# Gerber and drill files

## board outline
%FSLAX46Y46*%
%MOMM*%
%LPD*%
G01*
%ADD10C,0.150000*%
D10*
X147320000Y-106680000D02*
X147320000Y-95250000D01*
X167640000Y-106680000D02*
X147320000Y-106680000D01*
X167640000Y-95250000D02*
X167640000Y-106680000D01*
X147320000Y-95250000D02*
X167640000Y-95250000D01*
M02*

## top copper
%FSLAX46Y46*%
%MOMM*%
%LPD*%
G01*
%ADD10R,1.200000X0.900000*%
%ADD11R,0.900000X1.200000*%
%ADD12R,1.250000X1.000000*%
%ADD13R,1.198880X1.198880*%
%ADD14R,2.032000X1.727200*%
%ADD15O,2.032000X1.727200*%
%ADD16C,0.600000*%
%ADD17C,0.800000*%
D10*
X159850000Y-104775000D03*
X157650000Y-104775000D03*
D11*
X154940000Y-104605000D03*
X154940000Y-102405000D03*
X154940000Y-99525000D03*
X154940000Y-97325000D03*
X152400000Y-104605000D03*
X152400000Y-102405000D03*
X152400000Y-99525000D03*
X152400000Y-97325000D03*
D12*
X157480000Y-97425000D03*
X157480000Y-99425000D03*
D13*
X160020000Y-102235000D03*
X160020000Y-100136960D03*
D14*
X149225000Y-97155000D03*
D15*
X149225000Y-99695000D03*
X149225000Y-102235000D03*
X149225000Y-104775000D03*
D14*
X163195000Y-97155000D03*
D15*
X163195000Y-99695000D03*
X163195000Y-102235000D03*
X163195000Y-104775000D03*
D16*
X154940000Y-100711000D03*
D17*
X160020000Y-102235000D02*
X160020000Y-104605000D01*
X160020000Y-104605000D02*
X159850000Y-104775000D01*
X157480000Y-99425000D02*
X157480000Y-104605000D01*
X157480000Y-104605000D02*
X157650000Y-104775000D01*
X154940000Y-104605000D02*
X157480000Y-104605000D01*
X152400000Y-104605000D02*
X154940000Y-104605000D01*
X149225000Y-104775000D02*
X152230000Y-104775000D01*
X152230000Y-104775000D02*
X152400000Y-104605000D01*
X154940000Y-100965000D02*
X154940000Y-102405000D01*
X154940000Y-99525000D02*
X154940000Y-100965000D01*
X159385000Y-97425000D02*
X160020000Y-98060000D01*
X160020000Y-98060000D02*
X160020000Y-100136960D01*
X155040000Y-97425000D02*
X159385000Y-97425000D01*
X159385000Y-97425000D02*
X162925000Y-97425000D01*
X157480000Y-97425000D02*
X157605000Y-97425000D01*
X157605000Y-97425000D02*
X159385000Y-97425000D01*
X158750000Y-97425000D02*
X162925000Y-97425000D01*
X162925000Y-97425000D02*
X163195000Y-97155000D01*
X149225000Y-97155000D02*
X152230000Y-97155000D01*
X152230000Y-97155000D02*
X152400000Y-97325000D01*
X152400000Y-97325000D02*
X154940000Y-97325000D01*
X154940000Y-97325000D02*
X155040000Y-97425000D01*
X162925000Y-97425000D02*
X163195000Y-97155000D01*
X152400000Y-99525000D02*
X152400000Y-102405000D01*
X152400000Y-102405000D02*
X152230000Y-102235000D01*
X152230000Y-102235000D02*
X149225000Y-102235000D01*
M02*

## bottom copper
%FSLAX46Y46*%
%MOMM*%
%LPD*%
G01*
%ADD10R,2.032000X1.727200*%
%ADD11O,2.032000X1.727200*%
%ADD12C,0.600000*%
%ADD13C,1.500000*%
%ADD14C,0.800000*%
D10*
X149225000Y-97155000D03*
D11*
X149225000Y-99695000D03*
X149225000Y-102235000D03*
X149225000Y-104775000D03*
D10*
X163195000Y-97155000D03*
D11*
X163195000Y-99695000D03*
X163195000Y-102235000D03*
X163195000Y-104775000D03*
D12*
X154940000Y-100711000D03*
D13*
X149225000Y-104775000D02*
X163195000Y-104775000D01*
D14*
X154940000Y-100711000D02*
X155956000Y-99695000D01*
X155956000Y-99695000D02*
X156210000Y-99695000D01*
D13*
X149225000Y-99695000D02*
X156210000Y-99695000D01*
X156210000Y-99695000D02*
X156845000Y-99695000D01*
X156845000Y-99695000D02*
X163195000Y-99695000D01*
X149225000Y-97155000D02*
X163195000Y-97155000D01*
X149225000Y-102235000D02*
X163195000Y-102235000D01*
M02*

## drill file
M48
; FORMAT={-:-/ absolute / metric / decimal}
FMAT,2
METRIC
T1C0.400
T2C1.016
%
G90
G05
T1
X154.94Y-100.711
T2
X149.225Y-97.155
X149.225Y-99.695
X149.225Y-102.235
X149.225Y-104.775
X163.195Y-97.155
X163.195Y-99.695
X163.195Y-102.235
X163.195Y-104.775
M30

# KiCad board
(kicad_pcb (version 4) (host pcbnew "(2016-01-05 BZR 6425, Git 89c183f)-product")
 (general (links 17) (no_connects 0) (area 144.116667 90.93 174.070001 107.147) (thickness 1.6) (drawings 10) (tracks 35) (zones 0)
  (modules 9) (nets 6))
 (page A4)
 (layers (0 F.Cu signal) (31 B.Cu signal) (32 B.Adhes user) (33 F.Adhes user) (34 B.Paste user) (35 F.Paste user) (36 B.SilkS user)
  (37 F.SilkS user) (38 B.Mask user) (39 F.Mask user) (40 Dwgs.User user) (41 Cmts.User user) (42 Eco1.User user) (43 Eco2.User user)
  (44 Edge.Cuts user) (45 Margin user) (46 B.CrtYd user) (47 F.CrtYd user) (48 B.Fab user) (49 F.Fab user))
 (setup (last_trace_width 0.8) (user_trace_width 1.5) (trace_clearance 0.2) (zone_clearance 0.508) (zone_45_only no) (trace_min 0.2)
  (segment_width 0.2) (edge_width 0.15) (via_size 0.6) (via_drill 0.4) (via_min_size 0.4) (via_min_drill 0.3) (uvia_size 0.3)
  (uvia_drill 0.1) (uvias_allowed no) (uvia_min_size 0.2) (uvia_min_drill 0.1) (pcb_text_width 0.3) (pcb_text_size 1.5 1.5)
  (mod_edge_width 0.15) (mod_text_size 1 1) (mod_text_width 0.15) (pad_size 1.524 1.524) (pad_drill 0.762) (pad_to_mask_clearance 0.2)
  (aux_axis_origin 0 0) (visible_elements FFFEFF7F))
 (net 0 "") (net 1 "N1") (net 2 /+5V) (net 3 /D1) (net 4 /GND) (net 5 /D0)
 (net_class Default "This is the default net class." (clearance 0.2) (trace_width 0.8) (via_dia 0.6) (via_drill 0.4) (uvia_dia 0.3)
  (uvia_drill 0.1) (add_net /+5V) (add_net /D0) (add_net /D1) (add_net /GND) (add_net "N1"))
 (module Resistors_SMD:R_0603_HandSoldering (layer F.Cu) (at 158.75 104.775 180)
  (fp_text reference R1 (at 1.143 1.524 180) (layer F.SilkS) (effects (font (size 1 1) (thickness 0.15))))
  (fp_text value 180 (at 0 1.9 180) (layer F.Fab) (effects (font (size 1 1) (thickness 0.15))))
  (pad 1 smd rect (at -1.1 0 180) (size 1.2 0.9) (layers F.Cu F.Paste F.Mask) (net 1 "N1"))
  (pad 2 smd rect (at 1.1 0 180) (size 1.2 0.9) (layers F.Cu F.Paste F.Mask) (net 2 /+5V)))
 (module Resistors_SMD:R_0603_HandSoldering (layer F.Cu) (at 154.94 103.505 90)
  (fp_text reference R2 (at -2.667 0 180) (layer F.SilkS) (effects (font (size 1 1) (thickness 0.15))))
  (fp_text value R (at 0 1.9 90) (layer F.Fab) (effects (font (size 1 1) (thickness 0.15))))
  (pad 1 smd rect (at -1.1 0 90) (size 1.2 0.9) (layers F.Cu F.Paste F.Mask) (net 2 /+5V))
  (pad 2 smd rect (at 1.1 0 90) (size 1.2 0.9) (layers F.Cu F.Paste F.Mask) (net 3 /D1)))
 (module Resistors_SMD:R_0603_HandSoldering (layer F.Cu) (at 154.94 98.425 90)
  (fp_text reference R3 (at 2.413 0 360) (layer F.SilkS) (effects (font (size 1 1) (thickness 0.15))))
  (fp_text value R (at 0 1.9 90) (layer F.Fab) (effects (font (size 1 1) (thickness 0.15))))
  (pad 1 smd rect (at -1.1 0 90) (size 1.2 0.9) (layers F.Cu F.Paste F.Mask) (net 3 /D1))
  (pad 2 smd rect (at 1.1 0 90) (size 1.2 0.9) (layers F.Cu F.Paste F.Mask) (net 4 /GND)))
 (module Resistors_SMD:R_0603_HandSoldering (layer F.Cu) (at 152.4 103.505 90)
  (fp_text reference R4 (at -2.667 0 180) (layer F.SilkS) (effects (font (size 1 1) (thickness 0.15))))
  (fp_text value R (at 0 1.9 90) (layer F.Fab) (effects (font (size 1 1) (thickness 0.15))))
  (pad 1 smd rect (at -1.1 0 90) (size 1.2 0.9) (layers F.Cu F.Paste F.Mask) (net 2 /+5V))
  (pad 2 smd rect (at 1.1 0 90) (size 1.2 0.9) (layers F.Cu F.Paste F.Mask) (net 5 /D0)))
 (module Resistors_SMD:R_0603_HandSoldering (layer F.Cu) (at 152.4 98.425 90)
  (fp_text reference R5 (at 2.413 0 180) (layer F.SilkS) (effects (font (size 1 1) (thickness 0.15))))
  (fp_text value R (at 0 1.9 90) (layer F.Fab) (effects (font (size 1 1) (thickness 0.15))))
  (pad 1 smd rect (at -1.1 0 90) (size 1.2 0.9) (layers F.Cu F.Paste F.Mask) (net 5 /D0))
  (pad 2 smd rect (at 1.1 0 90) (size 1.2 0.9) (layers F.Cu F.Paste F.Mask) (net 4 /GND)))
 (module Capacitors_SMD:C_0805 (layer F.Cu) (at 157.48 98.425 270)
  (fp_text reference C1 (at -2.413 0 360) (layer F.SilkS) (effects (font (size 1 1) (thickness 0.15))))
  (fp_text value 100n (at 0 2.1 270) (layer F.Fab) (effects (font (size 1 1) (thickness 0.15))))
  (pad 1 smd rect (at -1 0 270) (size 1 1.25) (layers F.Cu F.Paste F.Mask) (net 4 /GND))
  (pad 2 smd rect (at 1 0 270) (size 1 1.25) (layers F.Cu F.Paste F.Mask) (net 2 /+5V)))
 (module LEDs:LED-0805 (layer F.Cu) (at 160.02 101.18598 270)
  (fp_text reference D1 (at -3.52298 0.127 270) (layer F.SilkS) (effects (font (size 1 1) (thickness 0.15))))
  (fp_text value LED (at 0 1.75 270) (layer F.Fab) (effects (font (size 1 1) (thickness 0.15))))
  (pad 2 smd rect (at 1.04902 0 90) (size 1.19888 1.19888) (layers F.Cu F.Paste F.Mask) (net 1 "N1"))
  (pad 1 smd rect (at -1.04902 0 90) (size 1.19888 1.19888) (layers F.Cu F.Paste F.Mask) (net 4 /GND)))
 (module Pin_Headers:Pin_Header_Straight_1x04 (layer F.Cu) (at 149.225 97.155)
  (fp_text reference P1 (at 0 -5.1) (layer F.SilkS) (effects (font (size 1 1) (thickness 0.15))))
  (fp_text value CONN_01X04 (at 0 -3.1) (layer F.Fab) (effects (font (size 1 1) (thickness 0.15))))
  (pad 1 thru_hole rect (at 0 0) (size 2.032 1.7272) (drill 1.016) (layers *.Cu *.Mask F.SilkS) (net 4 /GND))
  (pad 2 thru_hole oval (at 0 2.54) (size 2.032 1.7272) (drill 1.016) (layers *.Cu *.Mask F.SilkS) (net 3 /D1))
  (pad 3 thru_hole oval (at 0 5.08) (size 2.032 1.7272) (drill 1.016) (layers *.Cu *.Mask F.SilkS) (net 5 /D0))
  (pad 4 thru_hole oval (at 0 7.62) (size 2.032 1.7272) (drill 1.016) (layers *.Cu *.Mask F.SilkS) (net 2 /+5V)))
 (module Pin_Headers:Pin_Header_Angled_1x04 (layer F.Cu) (at 163.195 97.155)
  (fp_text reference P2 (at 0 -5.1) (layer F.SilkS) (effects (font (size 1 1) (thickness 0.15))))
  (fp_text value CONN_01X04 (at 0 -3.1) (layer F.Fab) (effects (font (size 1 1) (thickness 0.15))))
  (pad 1 thru_hole rect (at 0 0) (size 2.032 1.7272) (drill 1.016) (layers *.Cu *.Mask F.SilkS) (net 4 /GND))
  (pad 2 thru_hole oval (at 0 2.54) (size 2.032 1.7272) (drill 1.016) (layers *.Cu *.Mask F.SilkS) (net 3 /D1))
  (pad 3 thru_hole oval (at 0 5.08) (size 2.032 1.7272) (drill 1.016) (layers *.Cu *.Mask F.SilkS) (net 5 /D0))
  (pad 4 thru_hole oval (at 0 7.62) (size 2.032 1.7272) (drill 1.016) (layers *.Cu *.Mask F.SilkS) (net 2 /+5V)))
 (gr_line (start 147.32 106.68) (end 147.32 95.25) (layer Edge.Cuts) (width 0.15))
 (gr_line (start 167.64 106.68) (end 147.32 106.68) (layer Edge.Cuts) (width 0.15))
 (gr_line (start 167.64 95.25) (end 167.64 106.68) (layer Edge.Cuts) (width 0.15))
 (gr_line (start 147.32 95.25) (end 167.64 95.25) (layer Edge.Cuts) (width 0.15))
 (segment (start 160.02 102.235) (end 160.02 104.605) (width 0.8) (layer F.Cu) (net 1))
 (segment (start 160.02 104.605) (end 159.85 104.775) (width 0.8) (layer F.Cu) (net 1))
 (segment (start 157.48 99.425) (end 157.48 104.605) (width 0.8) (layer F.Cu) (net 2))
 (segment (start 157.48 104.605) (end 157.65 104.775) (width 0.8) (layer F.Cu) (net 2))
 (segment (start 154.94 104.605) (end 157.48 104.605) (width 0.8) (layer F.Cu) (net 2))
 (segment (start 152.4 104.605) (end 154.94 104.605) (width 0.8) (layer F.Cu) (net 2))
 (segment (start 149.225 104.775) (end 152.23 104.775) (width 0.8) (layer F.Cu) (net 2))
 (segment (start 152.23 104.775) (end 152.4 104.605) (width 0.8) (layer F.Cu) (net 2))
 (segment (start 149.225 104.775) (end 163.195 104.775) (width 1.5) (layer B.Cu) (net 2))
 (segment (start 154.94 100.711) (end 155.956 99.695) (width 0.8) (layer B.Cu) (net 3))
 (segment (start 155.956 99.695) (end 156.21 99.695) (width 0.8) (layer B.Cu) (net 3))
 (segment (start 149.225 99.695) (end 156.21 99.695) (width 1.5) (layer B.Cu) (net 3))
 (segment (start 156.21 99.695) (end 156.845 99.695) (width 1.5) (layer B.Cu) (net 3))
 (segment (start 154.94 100.965) (end 154.94 102.405) (width 0.8) (layer F.Cu) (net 3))
 (segment (start 154.94 99.525) (end 154.94 100.965) (width 0.8) (layer F.Cu) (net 3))
 (via (at 154.94 100.711) (size 0.6) (drill 0.4) (layers F.Cu B.Cu) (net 3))
 (segment (start 156.845 99.695) (end 163.195 99.695) (width 1.5) (layer B.Cu) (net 3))
 (segment (start 159.385 97.425) (end 160.02 98.06) (width 0.8) (layer F.Cu) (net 4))
 (segment (start 160.02 98.06) (end 160.02 100.13696) (width 0.8) (layer F.Cu) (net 4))
 (segment (start 155.04 97.425) (end 159.385 97.425) (width 0.8) (layer F.Cu) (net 4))
 (segment (start 159.385 97.425) (end 162.925 97.425) (width 0.8) (layer F.Cu) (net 4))
 (segment (start 157.48 97.425) (end 157.605 97.425) (width 0.8) (layer F.Cu) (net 4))
 (segment (start 157.605 97.425) (end 159.385 97.425) (width 0.8) (layer F.Cu) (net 4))
 (segment (start 158.75 97.425) (end 162.925 97.425) (width 0.8) (layer F.Cu) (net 4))
 (segment (start 162.925 97.425) (end 163.195 97.155) (width 0.8) (layer F.Cu) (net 4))
 (segment (start 149.225 97.155) (end 152.23 97.155) (width 0.8) (layer F.Cu) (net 4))
 (segment (start 152.23 97.155) (end 152.4 97.325) (width 0.8) (layer F.Cu) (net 4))
 (segment (start 152.4 97.325) (end 154.94 97.325) (width 0.8) (layer F.Cu) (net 4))
 (segment (start 154.94 97.325) (end 155.04 97.425) (width 0.8) (layer F.Cu) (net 4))
 (segment (start 162.925 97.425) (end 163.195 97.155) (width 0.8) (layer F.Cu) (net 4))
 (segment (start 149.225 97.155) (end 163.195 97.155) (width 1.5) (layer B.Cu) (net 4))
 (segment (start 152.4 99.525) (end 152.4 102.405) (width 0.8) (layer F.Cu) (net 5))
 (segment (start 152.4 102.405) (end 152.23 102.235) (width 0.8) (layer F.Cu) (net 5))
 (segment (start 152.23 102.235) (end 149.225 102.235) (width 0.8) (layer F.Cu) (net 5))
 (segment (start 149.225 102.235) (end 163.195 102.235) (width 1.5) (layer B.Cu) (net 5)))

